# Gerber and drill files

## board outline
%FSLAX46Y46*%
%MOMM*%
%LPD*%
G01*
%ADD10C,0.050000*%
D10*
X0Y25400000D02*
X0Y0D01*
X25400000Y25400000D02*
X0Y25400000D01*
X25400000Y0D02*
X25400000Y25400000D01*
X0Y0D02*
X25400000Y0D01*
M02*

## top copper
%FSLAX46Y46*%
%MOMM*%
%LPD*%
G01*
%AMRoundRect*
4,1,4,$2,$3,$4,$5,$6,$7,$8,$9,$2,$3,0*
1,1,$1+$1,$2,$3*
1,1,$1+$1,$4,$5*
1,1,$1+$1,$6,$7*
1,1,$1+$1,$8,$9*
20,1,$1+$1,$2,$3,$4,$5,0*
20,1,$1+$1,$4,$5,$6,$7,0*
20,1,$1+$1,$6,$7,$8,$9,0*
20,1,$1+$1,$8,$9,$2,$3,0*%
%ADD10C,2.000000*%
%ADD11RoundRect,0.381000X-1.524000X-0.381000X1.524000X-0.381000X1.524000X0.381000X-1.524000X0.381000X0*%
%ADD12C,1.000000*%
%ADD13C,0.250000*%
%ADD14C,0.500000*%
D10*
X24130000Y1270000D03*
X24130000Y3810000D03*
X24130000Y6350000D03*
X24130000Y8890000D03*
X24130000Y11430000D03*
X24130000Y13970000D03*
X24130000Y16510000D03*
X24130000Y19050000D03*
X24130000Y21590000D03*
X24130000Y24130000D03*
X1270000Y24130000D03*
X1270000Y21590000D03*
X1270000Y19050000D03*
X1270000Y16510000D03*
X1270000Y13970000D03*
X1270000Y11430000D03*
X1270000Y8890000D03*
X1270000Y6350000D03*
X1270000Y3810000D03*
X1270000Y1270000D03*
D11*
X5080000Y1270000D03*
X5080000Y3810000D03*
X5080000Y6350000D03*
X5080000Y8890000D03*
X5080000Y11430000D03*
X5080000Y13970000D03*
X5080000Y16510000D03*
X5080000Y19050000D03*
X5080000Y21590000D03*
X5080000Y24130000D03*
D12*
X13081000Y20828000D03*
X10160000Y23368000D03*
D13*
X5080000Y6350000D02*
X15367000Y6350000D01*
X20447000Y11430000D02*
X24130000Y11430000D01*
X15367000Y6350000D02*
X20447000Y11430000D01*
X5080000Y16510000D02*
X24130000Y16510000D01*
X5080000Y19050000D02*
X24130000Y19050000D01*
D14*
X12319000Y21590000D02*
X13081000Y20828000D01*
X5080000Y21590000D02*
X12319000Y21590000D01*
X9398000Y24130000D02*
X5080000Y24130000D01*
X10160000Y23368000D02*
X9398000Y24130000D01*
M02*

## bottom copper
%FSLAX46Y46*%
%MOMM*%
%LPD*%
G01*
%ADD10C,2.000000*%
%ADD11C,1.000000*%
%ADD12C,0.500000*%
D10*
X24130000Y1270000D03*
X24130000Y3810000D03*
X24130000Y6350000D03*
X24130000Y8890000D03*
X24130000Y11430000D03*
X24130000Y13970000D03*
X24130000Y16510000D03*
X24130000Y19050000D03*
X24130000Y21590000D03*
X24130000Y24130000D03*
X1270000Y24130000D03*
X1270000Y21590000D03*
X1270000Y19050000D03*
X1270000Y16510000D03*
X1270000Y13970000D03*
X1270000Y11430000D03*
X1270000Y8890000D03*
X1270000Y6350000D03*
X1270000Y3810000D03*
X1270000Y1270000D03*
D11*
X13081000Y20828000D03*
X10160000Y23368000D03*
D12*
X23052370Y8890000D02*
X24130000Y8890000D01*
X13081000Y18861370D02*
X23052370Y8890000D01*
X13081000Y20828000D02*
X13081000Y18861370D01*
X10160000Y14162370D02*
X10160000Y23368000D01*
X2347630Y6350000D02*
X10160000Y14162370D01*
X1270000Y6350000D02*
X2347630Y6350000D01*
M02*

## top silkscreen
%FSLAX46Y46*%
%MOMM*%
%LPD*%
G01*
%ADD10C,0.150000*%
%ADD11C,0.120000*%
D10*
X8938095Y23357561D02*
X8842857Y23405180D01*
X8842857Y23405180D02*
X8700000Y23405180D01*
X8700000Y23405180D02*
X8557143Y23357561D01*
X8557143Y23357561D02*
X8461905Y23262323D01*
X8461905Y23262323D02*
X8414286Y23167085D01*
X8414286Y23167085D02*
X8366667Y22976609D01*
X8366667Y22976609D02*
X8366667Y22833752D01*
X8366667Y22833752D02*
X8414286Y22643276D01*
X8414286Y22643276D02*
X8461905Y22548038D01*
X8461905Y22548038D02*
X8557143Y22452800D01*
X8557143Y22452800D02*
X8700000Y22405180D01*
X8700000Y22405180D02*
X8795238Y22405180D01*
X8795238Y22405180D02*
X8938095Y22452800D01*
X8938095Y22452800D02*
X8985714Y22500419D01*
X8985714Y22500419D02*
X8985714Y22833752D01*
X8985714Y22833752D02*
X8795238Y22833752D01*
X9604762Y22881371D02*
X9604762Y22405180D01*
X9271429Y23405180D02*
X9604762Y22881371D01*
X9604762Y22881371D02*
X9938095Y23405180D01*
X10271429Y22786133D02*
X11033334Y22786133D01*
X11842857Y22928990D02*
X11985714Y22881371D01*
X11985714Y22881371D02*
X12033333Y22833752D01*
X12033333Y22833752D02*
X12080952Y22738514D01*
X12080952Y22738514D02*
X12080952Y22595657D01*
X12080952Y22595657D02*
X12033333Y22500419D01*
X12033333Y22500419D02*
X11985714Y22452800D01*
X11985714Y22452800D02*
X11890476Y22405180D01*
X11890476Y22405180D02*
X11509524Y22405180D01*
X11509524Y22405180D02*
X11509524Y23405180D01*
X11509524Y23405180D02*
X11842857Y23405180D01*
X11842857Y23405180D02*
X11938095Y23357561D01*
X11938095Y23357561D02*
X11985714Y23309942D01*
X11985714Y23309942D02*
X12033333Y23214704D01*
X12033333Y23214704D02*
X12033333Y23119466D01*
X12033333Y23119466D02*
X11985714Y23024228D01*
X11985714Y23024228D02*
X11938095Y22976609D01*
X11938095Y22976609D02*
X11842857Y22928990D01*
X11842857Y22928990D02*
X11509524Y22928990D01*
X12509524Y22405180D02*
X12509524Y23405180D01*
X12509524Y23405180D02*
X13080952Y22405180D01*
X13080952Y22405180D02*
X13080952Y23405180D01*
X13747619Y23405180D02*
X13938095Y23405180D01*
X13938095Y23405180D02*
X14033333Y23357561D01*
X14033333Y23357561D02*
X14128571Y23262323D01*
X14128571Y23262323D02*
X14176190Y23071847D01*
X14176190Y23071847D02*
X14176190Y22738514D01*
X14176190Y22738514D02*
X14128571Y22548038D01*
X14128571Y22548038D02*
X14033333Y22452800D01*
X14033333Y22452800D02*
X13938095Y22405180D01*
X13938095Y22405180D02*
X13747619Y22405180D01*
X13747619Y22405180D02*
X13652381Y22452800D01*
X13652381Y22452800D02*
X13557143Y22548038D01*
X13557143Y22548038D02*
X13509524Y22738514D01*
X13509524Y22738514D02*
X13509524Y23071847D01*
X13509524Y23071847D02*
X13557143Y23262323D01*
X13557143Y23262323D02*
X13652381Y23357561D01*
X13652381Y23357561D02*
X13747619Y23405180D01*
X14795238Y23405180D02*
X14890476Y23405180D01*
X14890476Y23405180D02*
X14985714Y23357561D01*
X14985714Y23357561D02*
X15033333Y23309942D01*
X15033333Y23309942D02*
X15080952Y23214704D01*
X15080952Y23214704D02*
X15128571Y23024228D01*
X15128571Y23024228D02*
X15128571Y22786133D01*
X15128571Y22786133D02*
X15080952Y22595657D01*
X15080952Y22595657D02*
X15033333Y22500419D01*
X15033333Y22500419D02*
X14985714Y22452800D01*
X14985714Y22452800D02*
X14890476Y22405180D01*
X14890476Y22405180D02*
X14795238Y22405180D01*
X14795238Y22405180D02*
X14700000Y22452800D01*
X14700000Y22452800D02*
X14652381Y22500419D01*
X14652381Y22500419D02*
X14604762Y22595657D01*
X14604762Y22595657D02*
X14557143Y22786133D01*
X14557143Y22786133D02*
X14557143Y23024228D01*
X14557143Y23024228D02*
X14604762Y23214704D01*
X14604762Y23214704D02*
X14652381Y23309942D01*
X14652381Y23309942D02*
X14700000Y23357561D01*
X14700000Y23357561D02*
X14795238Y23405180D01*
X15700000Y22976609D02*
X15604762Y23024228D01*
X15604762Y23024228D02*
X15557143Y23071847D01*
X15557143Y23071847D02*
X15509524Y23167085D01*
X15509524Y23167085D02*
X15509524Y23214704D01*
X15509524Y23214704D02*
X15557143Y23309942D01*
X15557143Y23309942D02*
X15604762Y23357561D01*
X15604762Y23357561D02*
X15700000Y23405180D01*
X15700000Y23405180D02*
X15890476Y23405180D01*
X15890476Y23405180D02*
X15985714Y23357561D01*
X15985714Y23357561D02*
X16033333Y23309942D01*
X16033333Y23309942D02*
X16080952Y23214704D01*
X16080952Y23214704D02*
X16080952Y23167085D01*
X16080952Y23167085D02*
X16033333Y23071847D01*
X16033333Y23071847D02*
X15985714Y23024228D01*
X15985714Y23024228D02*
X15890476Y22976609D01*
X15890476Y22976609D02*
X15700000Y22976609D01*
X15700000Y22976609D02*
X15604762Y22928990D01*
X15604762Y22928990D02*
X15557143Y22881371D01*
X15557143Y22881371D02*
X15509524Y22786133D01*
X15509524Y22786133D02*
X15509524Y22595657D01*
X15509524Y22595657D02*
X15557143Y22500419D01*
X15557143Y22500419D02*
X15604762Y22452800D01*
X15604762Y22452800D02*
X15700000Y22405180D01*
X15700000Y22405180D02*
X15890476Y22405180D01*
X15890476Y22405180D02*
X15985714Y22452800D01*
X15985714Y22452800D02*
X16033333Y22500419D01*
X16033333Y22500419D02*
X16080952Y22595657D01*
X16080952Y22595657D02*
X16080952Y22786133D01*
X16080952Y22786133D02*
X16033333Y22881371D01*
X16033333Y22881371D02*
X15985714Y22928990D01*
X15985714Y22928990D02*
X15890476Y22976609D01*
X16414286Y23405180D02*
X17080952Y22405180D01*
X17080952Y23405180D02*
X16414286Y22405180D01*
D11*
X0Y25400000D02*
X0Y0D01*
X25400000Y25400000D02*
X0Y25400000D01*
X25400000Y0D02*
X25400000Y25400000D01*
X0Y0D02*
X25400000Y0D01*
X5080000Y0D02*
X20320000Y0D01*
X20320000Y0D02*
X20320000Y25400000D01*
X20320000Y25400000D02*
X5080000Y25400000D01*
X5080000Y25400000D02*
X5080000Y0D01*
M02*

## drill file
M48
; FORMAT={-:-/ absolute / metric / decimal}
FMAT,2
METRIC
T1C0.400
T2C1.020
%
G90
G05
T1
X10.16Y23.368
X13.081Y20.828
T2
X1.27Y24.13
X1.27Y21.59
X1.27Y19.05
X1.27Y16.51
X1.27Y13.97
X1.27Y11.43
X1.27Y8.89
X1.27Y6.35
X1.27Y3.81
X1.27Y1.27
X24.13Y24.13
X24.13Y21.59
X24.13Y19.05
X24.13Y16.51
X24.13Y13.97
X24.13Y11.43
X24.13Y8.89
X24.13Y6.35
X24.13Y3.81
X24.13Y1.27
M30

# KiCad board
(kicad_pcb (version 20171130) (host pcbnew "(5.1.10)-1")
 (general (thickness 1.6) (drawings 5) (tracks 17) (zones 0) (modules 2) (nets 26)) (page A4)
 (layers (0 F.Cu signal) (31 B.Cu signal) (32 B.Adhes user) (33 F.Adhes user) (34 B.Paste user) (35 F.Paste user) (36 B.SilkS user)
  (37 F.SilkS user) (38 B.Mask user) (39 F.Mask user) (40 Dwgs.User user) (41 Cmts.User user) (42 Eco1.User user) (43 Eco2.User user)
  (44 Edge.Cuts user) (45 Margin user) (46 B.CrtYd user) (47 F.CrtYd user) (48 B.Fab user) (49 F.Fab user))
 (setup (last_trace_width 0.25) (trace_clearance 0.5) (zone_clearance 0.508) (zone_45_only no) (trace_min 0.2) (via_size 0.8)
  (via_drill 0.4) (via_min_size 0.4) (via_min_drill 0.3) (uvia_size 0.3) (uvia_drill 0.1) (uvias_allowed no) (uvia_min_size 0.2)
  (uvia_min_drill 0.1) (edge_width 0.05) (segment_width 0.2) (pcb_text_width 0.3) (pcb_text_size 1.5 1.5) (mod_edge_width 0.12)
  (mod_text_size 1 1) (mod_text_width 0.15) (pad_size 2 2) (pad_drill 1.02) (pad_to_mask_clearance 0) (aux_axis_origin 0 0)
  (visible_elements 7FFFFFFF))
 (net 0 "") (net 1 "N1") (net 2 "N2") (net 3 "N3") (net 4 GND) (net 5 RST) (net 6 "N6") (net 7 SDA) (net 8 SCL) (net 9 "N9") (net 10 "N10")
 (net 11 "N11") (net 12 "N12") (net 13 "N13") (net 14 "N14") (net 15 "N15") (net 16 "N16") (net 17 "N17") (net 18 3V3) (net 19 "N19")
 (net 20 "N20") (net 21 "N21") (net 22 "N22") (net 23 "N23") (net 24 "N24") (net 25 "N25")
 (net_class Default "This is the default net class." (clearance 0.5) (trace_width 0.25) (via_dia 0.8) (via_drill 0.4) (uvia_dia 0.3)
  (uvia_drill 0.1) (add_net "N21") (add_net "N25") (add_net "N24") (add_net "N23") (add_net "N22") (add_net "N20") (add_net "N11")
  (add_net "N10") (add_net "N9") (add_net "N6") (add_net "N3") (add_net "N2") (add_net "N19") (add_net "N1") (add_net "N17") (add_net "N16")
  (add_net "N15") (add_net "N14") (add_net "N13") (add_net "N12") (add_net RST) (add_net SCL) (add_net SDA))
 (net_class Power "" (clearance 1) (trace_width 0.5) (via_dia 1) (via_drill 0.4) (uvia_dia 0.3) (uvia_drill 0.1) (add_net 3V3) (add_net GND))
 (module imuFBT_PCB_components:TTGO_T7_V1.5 (layer F.Cu) (at 0 0)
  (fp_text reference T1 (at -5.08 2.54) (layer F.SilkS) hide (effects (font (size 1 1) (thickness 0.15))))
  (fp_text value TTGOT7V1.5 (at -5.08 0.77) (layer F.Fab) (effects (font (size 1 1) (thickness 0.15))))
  (fp_line (start 0 -25.4) (end 0 0) (layer F.SilkS) (width 0.12))
  (fp_line (start 25.4 -25.4) (end 0 -25.4) (layer F.SilkS) (width 0.12))
  (fp_line (start 25.4 0) (end 25.4 -25.4) (layer F.SilkS) (width 0.12))
  (fp_line (start 0 0) (end 25.4 0) (layer F.SilkS) (width 0.12))
  (pad 20 thru_hole circle (at 24.13 -1.27) (size 2 2) (drill 1.02) (layers *.Cu *.Mask) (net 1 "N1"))
  (pad 19 thru_hole circle (at 24.13 -3.81) (size 2 2) (drill 1.02) (layers *.Cu *.Mask) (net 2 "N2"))
  (pad 18 thru_hole circle (at 24.13 -6.35) (size 2 2) (drill 1.02) (layers *.Cu *.Mask) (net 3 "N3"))
  (pad 17 thru_hole circle (at 24.13 -8.89) (size 2 2) (drill 1.02) (layers *.Cu *.Mask) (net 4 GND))
  (pad 16 thru_hole circle (at 24.13 -11.43) (size 2 2) (drill 1.02) (layers *.Cu *.Mask) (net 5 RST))
  (pad 15 thru_hole circle (at 24.13 -13.97) (size 2 2) (drill 1.02) (layers *.Cu *.Mask) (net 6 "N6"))
  (pad 14 thru_hole circle (at 24.13 -16.51) (size 2 2) (drill 1.02) (layers *.Cu *.Mask) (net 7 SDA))
  (pad 13 thru_hole circle (at 24.13 -19.05) (size 2 2) (drill 1.02) (layers *.Cu *.Mask) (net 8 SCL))
  (pad 12 thru_hole circle (at 24.13 -21.59) (size 2 2) (drill 1.02) (layers *.Cu *.Mask) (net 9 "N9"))
  (pad 11 thru_hole circle (at 24.13 -24.13) (size 2 2) (drill 1.02) (layers *.Cu *.Mask) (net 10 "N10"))
  (pad 10 thru_hole circle (at 1.27 -24.13) (size 2 2) (drill 1.02) (layers *.Cu *.Mask) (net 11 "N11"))
  (pad 9 thru_hole circle (at 1.27 -21.59) (size 2 2) (drill 1.02) (layers *.Cu *.Mask) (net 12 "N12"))
  (pad 8 thru_hole circle (at 1.27 -19.05) (size 2 2) (drill 1.02) (layers *.Cu *.Mask) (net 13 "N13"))
  (pad 7 thru_hole circle (at 1.27 -16.51) (size 2 2) (drill 1.02) (layers *.Cu *.Mask) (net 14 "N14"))
  (pad 6 thru_hole circle (at 1.27 -13.97) (size 2 2) (drill 1.02) (layers *.Cu *.Mask) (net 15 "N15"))
  (pad 5 thru_hole circle (at 1.27 -11.43) (size 2 2) (drill 1.02) (layers *.Cu *.Mask) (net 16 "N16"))
  (pad 4 thru_hole circle (at 1.27 -8.89) (size 2 2) (drill 1.02) (layers *.Cu *.Mask) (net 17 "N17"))
  (pad 3 thru_hole circle (at 1.27 -6.35) (size 2 2) (drill 1.02) (layers *.Cu *.Mask) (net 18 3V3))
  (pad 2 thru_hole circle (at 1.27 -3.81) (size 2 2) (drill 1.02) (layers *.Cu *.Mask) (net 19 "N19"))
  (pad 1 thru_hole circle (at 1.27 -1.27) (size 2 2) (drill 1.02) (layers *.Cu *.Mask) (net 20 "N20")))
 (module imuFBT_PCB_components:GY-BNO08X (layer F.Cu) (at 5.08 0)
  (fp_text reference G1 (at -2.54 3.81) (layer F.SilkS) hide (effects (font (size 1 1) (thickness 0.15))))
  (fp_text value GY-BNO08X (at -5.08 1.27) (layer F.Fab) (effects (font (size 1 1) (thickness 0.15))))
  (fp_line (start 0 0) (end 15.24 0) (layer F.SilkS) (width 0.12))
  (fp_line (start 15.24 0) (end 15.24 -25.4) (layer F.SilkS) (width 0.12))
  (fp_line (start 15.24 -25.4) (end 0 -25.4) (layer F.SilkS) (width 0.12))
  (fp_line (start 0 -25.4) (end 0 0) (layer F.SilkS) (width 0.12))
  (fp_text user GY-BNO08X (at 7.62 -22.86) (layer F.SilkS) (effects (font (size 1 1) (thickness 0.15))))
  (pad 10 smd roundrect (at 0 -1.27) (size 3.81 1.524) (layers F.Cu F.Paste F.Mask) (roundrect_rratio 0.25) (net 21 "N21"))
  (pad 9 smd roundrect (at 0 -3.81) (size 3.81 1.524) (layers F.Cu F.Paste F.Mask) (roundrect_rratio 0.25) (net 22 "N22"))
  (pad 8 smd roundrect (at 0 -6.35) (size 3.81 1.524) (layers F.Cu F.Paste F.Mask) (roundrect_rratio 0.25) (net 5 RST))
  (pad 7 smd roundrect (at 0 -8.89) (size 3.81 1.524) (layers F.Cu F.Paste F.Mask) (roundrect_rratio 0.25) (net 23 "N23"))
  (pad 6 smd roundrect (at 0 -11.43) (size 3.81 1.524) (layers F.Cu F.Paste F.Mask) (roundrect_rratio 0.25) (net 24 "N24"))
  (pad 5 smd roundrect (at 0 -13.97) (size 3.81 1.524) (layers F.Cu F.Paste F.Mask) (roundrect_rratio 0.25) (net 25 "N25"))
  (pad 4 smd roundrect (at 0 -16.51) (size 3.81 1.524) (layers F.Cu F.Paste F.Mask) (roundrect_rratio 0.25) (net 7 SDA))
  (pad 3 smd roundrect (at 0 -19.05) (size 3.81 1.524) (layers F.Cu F.Paste F.Mask) (roundrect_rratio 0.25) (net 8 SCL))
  (pad 2 smd roundrect (at 0 -21.59) (size 3.81 1.524) (layers F.Cu F.Paste F.Mask) (roundrect_rratio 0.25) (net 4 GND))
  (pad 1 smd roundrect (at 0 -24.13) (size 3.81 1.524) (layers F.Cu F.Paste F.Mask) (roundrect_rratio 0.25) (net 18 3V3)))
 (gr_line (start 0 -25.4) (end 0 0) (layer Edge.Cuts) (width 0.05))
 (gr_line (start 25.4 -25.4) (end 0 -25.4) (layer Edge.Cuts) (width 0.05))
 (gr_line (start 25.4 0) (end 25.4 -25.4) (layer Edge.Cuts) (width 0.05))
 (gr_line (start 0 0) (end 25.4 0) (layer Edge.Cuts) (width 0.05))
 (segment (start 5.08 -6.35) (end 15.367 -6.35) (width 0.25) (layer F.Cu) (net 5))
 (segment (start 20.447 -11.43) (end 24.13 -11.43) (width 0.25) (layer F.Cu) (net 5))
 (segment (start 15.367 -6.35) (end 20.447 -11.43) (width 0.25) (layer F.Cu) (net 5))
 (segment (start 5.08 -16.51) (end 24.13 -16.51) (width 0.25) (layer F.Cu) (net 7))
 (segment (start 5.08 -19.05) (end 24.13 -19.05) (width 0.25) (layer F.Cu) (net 8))
 (via (at 13.081 -20.828) (size 1) (drill 0.4) (layers F.Cu B.Cu) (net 4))
 (segment (start 12.319 -21.59) (end 13.081 -20.828) (width 0.5) (layer F.Cu) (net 4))
 (segment (start 5.08 -21.59) (end 12.319 -21.59) (width 0.5) (layer F.Cu) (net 4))
 (segment (start 23.05237 -8.89) (end 24.13 -8.89) (width 0.5) (layer B.Cu) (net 4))
 (segment (start 13.081 -18.86137) (end 23.05237 -8.89) (width 0.5) (layer B.Cu) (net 4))
 (segment (start 13.081 -20.828) (end 13.081 -18.86137) (width 0.5) (layer B.Cu) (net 4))
 (via (at 10.16 -23.368) (size 1) (drill 0.4) (layers F.Cu B.Cu) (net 18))
 (segment (start 10.16 -14.16237) (end 10.16 -23.368) (width 0.5) (layer B.Cu) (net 18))
 (segment (start 2.34763 -6.35) (end 10.16 -14.16237) (width 0.5) (layer B.Cu) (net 18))
 (segment (start 1.27 -6.35) (end 2.34763 -6.35) (width 0.5) (layer B.Cu) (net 18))
 (segment (start 9.398 -24.13) (end 5.08 -24.13) (width 0.5) (layer F.Cu) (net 18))
 (segment (start 10.16 -23.368) (end 9.398 -24.13) (width 0.5) (layer F.Cu) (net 18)))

